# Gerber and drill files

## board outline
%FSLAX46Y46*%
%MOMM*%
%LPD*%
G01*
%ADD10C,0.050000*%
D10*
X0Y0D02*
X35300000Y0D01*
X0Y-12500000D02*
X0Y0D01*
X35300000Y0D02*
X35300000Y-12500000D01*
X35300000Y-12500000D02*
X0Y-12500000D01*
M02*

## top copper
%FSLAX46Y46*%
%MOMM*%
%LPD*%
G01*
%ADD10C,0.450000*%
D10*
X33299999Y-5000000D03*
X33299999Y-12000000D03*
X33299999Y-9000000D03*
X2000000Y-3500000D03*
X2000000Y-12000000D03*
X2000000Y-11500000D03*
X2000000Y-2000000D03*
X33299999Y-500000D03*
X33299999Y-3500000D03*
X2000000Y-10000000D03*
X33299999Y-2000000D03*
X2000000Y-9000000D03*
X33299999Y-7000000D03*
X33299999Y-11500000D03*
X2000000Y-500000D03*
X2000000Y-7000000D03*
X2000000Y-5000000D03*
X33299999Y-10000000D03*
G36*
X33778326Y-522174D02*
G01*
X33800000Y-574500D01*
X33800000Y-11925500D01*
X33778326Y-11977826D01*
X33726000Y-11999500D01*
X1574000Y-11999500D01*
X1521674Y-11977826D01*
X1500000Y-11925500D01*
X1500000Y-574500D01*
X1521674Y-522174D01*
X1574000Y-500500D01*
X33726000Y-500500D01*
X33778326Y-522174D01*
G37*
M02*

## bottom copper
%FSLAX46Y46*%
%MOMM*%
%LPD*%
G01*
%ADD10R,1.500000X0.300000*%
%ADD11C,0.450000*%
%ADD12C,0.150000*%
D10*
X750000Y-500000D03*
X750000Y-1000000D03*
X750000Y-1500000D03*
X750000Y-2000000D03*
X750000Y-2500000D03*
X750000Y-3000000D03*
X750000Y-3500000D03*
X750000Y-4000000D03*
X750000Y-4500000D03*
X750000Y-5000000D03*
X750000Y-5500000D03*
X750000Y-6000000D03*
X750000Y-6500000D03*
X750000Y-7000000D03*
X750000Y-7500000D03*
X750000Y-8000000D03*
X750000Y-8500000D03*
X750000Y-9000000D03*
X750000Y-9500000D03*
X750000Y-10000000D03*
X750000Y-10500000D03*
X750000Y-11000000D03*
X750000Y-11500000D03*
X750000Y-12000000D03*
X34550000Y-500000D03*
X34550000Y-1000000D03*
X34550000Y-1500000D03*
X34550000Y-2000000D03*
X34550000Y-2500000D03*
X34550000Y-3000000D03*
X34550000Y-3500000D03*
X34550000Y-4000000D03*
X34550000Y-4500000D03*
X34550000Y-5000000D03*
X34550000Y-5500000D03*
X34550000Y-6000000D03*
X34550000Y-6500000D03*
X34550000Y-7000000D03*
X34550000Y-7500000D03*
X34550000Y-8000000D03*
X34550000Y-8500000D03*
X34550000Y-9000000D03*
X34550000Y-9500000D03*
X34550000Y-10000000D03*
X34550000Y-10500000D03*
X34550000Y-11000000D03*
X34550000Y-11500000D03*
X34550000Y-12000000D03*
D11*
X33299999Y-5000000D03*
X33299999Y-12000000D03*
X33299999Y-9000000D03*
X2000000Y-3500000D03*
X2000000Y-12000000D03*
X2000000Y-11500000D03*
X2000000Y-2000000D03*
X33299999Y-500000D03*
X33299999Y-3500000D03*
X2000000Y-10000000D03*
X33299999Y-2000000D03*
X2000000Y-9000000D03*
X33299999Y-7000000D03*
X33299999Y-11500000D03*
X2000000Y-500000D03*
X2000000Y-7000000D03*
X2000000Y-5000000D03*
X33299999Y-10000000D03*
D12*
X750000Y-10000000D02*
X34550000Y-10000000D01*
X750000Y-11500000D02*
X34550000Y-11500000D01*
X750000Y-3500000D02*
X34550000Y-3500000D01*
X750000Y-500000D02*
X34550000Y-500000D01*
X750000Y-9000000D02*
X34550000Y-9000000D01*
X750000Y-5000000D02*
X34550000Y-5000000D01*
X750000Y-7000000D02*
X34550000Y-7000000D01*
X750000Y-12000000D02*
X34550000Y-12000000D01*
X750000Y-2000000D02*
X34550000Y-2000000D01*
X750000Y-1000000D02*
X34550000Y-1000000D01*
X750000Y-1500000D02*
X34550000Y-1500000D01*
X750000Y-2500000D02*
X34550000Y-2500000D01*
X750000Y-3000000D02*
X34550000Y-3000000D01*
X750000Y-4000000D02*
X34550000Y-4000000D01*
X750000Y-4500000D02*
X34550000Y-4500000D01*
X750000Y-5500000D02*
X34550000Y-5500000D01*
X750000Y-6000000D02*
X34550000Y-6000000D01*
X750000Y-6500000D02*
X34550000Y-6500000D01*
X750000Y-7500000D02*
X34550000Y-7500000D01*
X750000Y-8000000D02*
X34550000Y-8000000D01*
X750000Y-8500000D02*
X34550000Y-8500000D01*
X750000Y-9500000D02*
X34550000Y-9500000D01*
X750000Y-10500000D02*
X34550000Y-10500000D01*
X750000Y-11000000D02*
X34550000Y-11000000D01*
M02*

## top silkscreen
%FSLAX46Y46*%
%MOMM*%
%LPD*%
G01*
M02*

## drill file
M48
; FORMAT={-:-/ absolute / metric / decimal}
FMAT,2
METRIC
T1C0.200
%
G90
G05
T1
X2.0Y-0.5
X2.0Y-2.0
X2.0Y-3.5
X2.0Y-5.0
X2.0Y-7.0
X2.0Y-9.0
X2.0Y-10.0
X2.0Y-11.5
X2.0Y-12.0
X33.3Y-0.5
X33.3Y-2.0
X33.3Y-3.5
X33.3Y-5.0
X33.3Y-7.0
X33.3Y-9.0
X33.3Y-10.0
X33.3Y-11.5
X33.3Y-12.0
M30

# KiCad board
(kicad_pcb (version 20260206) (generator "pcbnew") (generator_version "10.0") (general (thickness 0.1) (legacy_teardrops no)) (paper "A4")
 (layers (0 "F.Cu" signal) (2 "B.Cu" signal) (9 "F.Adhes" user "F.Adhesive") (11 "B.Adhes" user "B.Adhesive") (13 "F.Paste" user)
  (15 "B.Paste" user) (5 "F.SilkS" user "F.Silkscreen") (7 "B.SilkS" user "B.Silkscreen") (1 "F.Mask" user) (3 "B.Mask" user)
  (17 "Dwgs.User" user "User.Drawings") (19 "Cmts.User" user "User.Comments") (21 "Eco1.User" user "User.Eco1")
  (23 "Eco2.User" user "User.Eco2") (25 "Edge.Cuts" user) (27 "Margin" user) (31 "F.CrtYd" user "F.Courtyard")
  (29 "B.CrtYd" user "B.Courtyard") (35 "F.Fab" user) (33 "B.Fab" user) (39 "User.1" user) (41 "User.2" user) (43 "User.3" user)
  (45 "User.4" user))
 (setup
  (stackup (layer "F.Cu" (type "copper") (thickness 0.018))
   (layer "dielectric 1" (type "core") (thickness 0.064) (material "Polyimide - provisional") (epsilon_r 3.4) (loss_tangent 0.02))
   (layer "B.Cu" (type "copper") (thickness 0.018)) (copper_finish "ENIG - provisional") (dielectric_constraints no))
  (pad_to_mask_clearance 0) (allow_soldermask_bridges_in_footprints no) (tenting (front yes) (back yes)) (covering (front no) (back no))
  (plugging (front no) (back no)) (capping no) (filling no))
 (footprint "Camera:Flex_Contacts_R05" (layer "B.Cu") (at 0.75 6.25)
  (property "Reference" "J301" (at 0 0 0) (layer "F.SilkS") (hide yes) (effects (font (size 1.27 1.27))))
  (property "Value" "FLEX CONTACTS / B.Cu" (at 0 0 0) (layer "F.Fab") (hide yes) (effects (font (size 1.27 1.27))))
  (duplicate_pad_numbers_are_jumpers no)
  (pad "1" smd rect (at 0 -5.75) (size 1.5 0.3) (layers "B.Cu" "B.Mask") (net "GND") (thermal_bridge_angle 45))
  (pad "2" smd rect (at 0 -5.25) (size 1.5 0.3) (layers "B.Cu" "B.Mask") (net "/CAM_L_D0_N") (thermal_bridge_angle 45))
  (pad "3" smd rect (at 0 -4.75) (size 1.5 0.3) (layers "B.Cu" "B.Mask") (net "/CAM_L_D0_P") (thermal_bridge_angle 45))
  (pad "4" smd rect (at 0 -4.25) (size 1.5 0.3) (layers "B.Cu" "B.Mask") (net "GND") (thermal_bridge_angle 45))
  (pad "5" smd rect (at 0 -3.75) (size 1.5 0.3) (layers "B.Cu" "B.Mask") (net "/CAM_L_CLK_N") (thermal_bridge_angle 45))
  (pad "6" smd rect (at 0 -3.25) (size 1.5 0.3) (layers "B.Cu" "B.Mask") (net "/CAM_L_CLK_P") (thermal_bridge_angle 45))
  (pad "7" smd rect (at 0 -2.75) (size 1.5 0.3) (layers "B.Cu" "B.Mask") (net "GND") (thermal_bridge_angle 45))
  (pad "8" smd rect (at 0 -2.25) (size 1.5 0.3) (layers "B.Cu" "B.Mask") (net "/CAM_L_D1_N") (thermal_bridge_angle 45))
  (pad "9" smd rect (at 0 -1.75) (size 1.5 0.3) (layers "B.Cu" "B.Mask") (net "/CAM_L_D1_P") (thermal_bridge_angle 45))
  (pad "10" smd rect (at 0 -1.25) (size 1.5 0.3) (layers "B.Cu" "B.Mask") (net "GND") (thermal_bridge_angle 45))
  (pad "11" smd rect (at 0 -0.75) (size 1.5 0.3) (layers "B.Cu" "B.Mask") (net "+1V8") (thermal_bridge_angle 45))
  (pad "12" smd rect (at 0 -0.25) (size 1.5 0.3) (layers "B.Cu" "B.Mask") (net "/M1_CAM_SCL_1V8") (thermal_bridge_angle 45))
  (pad "13" smd rect (at 0 0.25) (size 1.5 0.3) (layers "B.Cu" "B.Mask") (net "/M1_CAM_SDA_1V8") (thermal_bridge_angle 45))
  (pad "14" smd rect (at 0 0.75) (size 1.5 0.3) (layers "B.Cu" "B.Mask") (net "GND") (thermal_bridge_angle 45))
  (pad "15" smd rect (at 0 1.25) (size 1.5 0.3) (layers "B.Cu" "B.Mask") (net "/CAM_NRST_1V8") (thermal_bridge_angle 45))
  (pad "16" smd rect (at 0 1.75) (size 1.5 0.3) (layers "B.Cu" "B.Mask") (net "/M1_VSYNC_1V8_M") (thermal_bridge_angle 45))
  (pad "17" smd rect (at 0 2.25) (size 1.5 0.3) (layers "B.Cu" "B.Mask") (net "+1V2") (thermal_bridge_angle 45))
  (pad "18" smd rect (at 0 2.75) (size 1.5 0.3) (layers "B.Cu" "B.Mask") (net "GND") (thermal_bridge_angle 45))
  (pad "19" smd rect (at 0 3.25) (size 1.5 0.3) (layers "B.Cu" "B.Mask") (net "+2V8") (thermal_bridge_angle 45))
  (pad "20" smd rect (at 0 3.75) (size 1.5 0.3) (layers "B.Cu" "B.Mask") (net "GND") (thermal_bridge_angle 45))
  (pad "21" smd rect (at 0 4.25) (size 1.5 0.3) (layers "B.Cu" "B.Mask") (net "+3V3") (thermal_bridge_angle 45))
  (pad "22" smd rect (at 0 4.75) (size 1.5 0.3) (layers "B.Cu" "B.Mask") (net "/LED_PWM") (thermal_bridge_angle 45))
  (pad "23" smd rect (at 0 5.25) (size 1.5 0.3) (layers "B.Cu" "B.Mask") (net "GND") (thermal_bridge_angle 45))
  (pad "24" smd rect (at 0 5.75) (size 1.5 0.3) (layers "B.Cu" "B.Mask") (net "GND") (thermal_bridge_angle 45)))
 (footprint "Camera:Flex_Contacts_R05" (layer "B.Cu") (at 34.55 6.25)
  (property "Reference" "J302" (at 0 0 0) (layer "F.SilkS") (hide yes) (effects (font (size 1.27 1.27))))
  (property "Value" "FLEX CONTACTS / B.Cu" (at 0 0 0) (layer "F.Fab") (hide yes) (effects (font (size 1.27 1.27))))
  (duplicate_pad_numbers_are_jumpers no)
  (pad "1" smd rect (at 0 -5.75) (size 1.5 0.3) (layers "B.Cu" "B.Mask") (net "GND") (thermal_bridge_angle 45))
  (pad "2" smd rect (at 0 -5.25) (size 1.5 0.3) (layers "B.Cu" "B.Mask") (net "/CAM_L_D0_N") (thermal_bridge_angle 45))
  (pad "3" smd rect (at 0 -4.75) (size 1.5 0.3) (layers "B.Cu" "B.Mask") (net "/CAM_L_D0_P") (thermal_bridge_angle 45))
  (pad "4" smd rect (at 0 -4.25) (size 1.5 0.3) (layers "B.Cu" "B.Mask") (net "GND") (thermal_bridge_angle 45))
  (pad "5" smd rect (at 0 -3.75) (size 1.5 0.3) (layers "B.Cu" "B.Mask") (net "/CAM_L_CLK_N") (thermal_bridge_angle 45))
  (pad "6" smd rect (at 0 -3.25) (size 1.5 0.3) (layers "B.Cu" "B.Mask") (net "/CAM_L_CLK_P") (thermal_bridge_angle 45))
  (pad "7" smd rect (at 0 -2.75) (size 1.5 0.3) (layers "B.Cu" "B.Mask") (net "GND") (thermal_bridge_angle 45))
  (pad "8" smd rect (at 0 -2.25) (size 1.5 0.3) (layers "B.Cu" "B.Mask") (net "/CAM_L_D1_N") (thermal_bridge_angle 45))
  (pad "9" smd rect (at 0 -1.75) (size 1.5 0.3) (layers "B.Cu" "B.Mask") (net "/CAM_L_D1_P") (thermal_bridge_angle 45))
  (pad "10" smd rect (at 0 -1.25) (size 1.5 0.3) (layers "B.Cu" "B.Mask") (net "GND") (thermal_bridge_angle 45))
  (pad "11" smd rect (at 0 -0.75) (size 1.5 0.3) (layers "B.Cu" "B.Mask") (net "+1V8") (thermal_bridge_angle 45))
  (pad "12" smd rect (at 0 -0.25) (size 1.5 0.3) (layers "B.Cu" "B.Mask") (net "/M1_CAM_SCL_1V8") (thermal_bridge_angle 45))
  (pad "13" smd rect (at 0 0.25) (size 1.5 0.3) (layers "B.Cu" "B.Mask") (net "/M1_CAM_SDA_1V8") (thermal_bridge_angle 45))
  (pad "14" smd rect (at 0 0.75) (size 1.5 0.3) (layers "B.Cu" "B.Mask") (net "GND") (thermal_bridge_angle 45))
  (pad "15" smd rect (at 0 1.25) (size 1.5 0.3) (layers "B.Cu" "B.Mask") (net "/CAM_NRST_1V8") (thermal_bridge_angle 45))
  (pad "16" smd rect (at 0 1.75) (size 1.5 0.3) (layers "B.Cu" "B.Mask") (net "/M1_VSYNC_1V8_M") (thermal_bridge_angle 45))
  (pad "17" smd rect (at 0 2.25) (size 1.5 0.3) (layers "B.Cu" "B.Mask") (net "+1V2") (thermal_bridge_angle 45))
  (pad "18" smd rect (at 0 2.75) (size 1.5 0.3) (layers "B.Cu" "B.Mask") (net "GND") (thermal_bridge_angle 45))
  (pad "19" smd rect (at 0 3.25) (size 1.5 0.3) (layers "B.Cu" "B.Mask") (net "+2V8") (thermal_bridge_angle 45))
  (pad "20" smd rect (at 0 3.75) (size 1.5 0.3) (layers "B.Cu" "B.Mask") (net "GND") (thermal_bridge_angle 45))
  (pad "21" smd rect (at 0 4.25) (size 1.5 0.3) (layers "B.Cu" "B.Mask") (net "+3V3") (thermal_bridge_angle 45))
  (pad "22" smd rect (at 0 4.75) (size 1.5 0.3) (layers "B.Cu" "B.Mask") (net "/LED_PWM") (thermal_bridge_angle 45))
  (pad "23" smd rect (at 0 5.25) (size 1.5 0.3) (layers "B.Cu" "B.Mask") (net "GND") (thermal_bridge_angle 45))
  (pad "24" smd rect (at 0 5.75) (size 1.5 0.3) (layers "B.Cu" "B.Mask") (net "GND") (thermal_bridge_angle 45)))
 (gr_line (start 0 0) (end 35.3 0) (stroke (width 0.05) (type default)) (layer "Edge.Cuts"))
 (gr_line (start 0 12.5) (end 0 0) (stroke (width 0.05) (type default)) (layer "Edge.Cuts"))
 (gr_line (start 35.3 0) (end 35.3 12.5) (stroke (width 0.05) (type default)) (layer "Edge.Cuts"))
 (gr_line (start 35.3 12.5) (end 0 12.5) (stroke (width 0.05) (type default)) (layer "Edge.Cuts"))
 (via (at 33.299999 5) (size 0.45) (drill 0.2) (layers "F.Cu" "B.Cu") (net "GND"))
 (via (at 33.299999 12) (size 0.45) (drill 0.2) (layers "F.Cu" "B.Cu") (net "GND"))
 (via (at 33.299999 9) (size 0.45) (drill 0.2) (layers "F.Cu" "B.Cu") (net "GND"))
 (via (at 2 3.5) (size 0.45) (drill 0.2) (layers "F.Cu" "B.Cu") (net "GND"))
 (via (at 2 12) (size 0.45) (drill 0.2) (layers "F.Cu" "B.Cu") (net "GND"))
 (via (at 2 11.5) (size 0.45) (drill 0.2) (layers "F.Cu" "B.Cu") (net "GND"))
 (via (at 2 2) (size 0.45) (drill 0.2) (layers "F.Cu" "B.Cu") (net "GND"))
 (via (at 33.299999 0.5) (size 0.45) (drill 0.2) (layers "F.Cu" "B.Cu") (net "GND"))
 (via (at 33.299999 3.5) (size 0.45) (drill 0.2) (layers "F.Cu" "B.Cu") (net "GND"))
 (via (at 2 10) (size 0.45) (drill 0.2) (layers "F.Cu" "B.Cu") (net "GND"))
 (via (at 33.299999 2) (size 0.45) (drill 0.2) (layers "F.Cu" "B.Cu") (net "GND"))
 (via (at 2 9) (size 0.45) (drill 0.2) (layers "F.Cu" "B.Cu") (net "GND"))
 (via (at 33.299999 7) (size 0.45) (drill 0.2) (layers "F.Cu" "B.Cu") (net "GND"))
 (via (at 33.299999 11.5) (size 0.45) (drill 0.2) (layers "F.Cu" "B.Cu") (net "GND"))
 (via (at 2 0.5) (size 0.45) (drill 0.2) (layers "F.Cu" "B.Cu") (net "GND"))
 (via (at 2 7) (size 0.45) (drill 0.2) (layers "F.Cu" "B.Cu") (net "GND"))
 (via (at 2 5) (size 0.45) (drill 0.2) (layers "F.Cu" "B.Cu") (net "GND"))
 (via (at 33.299999 10) (size 0.45) (drill 0.2) (layers "F.Cu" "B.Cu") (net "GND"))
 (segment (start 0.75 10) (end 34.55 10) (width 0.15) (layer "B.Cu") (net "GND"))
 (segment (start 0.75 11.5) (end 34.55 11.5) (width 0.15) (layer "B.Cu") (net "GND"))
 (segment (start 0.75 3.5) (end 34.55 3.5) (width 0.15) (layer "B.Cu") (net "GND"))
 (segment (start 0.75 0.5) (end 34.55 0.5) (width 0.15) (layer "B.Cu") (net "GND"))
 (segment (start 0.75 9) (end 34.55 9) (width 0.15) (layer "B.Cu") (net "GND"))
 (segment (start 0.75 5) (end 34.55 5) (width 0.15) (layer "B.Cu") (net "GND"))
 (segment (start 0.75 7) (end 34.55 7) (width 0.15) (layer "B.Cu") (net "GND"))
 (segment (start 0.75 12) (end 34.55 12) (width 0.15) (layer "B.Cu") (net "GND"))
 (segment (start 0.75 2) (end 34.55 2) (width 0.15) (layer "B.Cu") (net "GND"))
 (segment (start 0.75 1) (end 34.55 1) (width 0.15) (layer "B.Cu") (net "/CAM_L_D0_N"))
 (segment (start 0.75 1.5) (end 34.55 1.5) (width 0.15) (layer "B.Cu") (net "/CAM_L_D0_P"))
 (segment (start 0.75 2.5) (end 34.55 2.5) (width 0.15) (layer "B.Cu") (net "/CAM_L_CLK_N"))
 (segment (start 0.75 3) (end 34.55 3) (width 0.15) (layer "B.Cu") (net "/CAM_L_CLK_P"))
 (segment (start 0.75 4) (end 34.55 4) (width 0.15) (layer "B.Cu") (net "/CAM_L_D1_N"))
 (segment (start 0.75 4.5) (end 34.55 4.5) (width 0.15) (layer "B.Cu") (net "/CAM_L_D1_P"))
 (segment (start 0.75 5.5) (end 34.55 5.5) (width 0.15) (layer "B.Cu") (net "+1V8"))
 (segment (start 0.75 6) (end 34.55 6) (width 0.15) (layer "B.Cu") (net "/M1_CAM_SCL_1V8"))
 (segment (start 0.75 6.5) (end 34.55 6.5) (width 0.15) (layer "B.Cu") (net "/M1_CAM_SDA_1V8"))
 (segment (start 0.75 7.5) (end 34.55 7.5) (width 0.15) (layer "B.Cu") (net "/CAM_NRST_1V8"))
 (segment (start 0.75 8) (end 34.55 8) (width 0.15) (layer "B.Cu") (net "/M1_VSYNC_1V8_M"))
 (segment (start 0.75 8.5) (end 34.55 8.5) (width 0.15) (layer "B.Cu") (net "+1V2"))
 (segment (start 0.75 9.5) (end 34.55 9.5) (width 0.15) (layer "B.Cu") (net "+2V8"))
 (segment (start 0.75 10.5) (end 34.55 10.5) (width 0.15) (layer "B.Cu") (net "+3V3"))
 (segment (start 0.75 11) (end 34.55 11) (width 0.15) (layer "B.Cu") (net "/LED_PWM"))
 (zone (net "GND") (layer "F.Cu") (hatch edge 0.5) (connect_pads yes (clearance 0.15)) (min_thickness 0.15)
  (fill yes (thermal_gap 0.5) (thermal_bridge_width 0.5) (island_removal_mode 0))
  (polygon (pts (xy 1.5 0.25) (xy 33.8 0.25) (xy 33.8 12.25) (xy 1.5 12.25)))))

